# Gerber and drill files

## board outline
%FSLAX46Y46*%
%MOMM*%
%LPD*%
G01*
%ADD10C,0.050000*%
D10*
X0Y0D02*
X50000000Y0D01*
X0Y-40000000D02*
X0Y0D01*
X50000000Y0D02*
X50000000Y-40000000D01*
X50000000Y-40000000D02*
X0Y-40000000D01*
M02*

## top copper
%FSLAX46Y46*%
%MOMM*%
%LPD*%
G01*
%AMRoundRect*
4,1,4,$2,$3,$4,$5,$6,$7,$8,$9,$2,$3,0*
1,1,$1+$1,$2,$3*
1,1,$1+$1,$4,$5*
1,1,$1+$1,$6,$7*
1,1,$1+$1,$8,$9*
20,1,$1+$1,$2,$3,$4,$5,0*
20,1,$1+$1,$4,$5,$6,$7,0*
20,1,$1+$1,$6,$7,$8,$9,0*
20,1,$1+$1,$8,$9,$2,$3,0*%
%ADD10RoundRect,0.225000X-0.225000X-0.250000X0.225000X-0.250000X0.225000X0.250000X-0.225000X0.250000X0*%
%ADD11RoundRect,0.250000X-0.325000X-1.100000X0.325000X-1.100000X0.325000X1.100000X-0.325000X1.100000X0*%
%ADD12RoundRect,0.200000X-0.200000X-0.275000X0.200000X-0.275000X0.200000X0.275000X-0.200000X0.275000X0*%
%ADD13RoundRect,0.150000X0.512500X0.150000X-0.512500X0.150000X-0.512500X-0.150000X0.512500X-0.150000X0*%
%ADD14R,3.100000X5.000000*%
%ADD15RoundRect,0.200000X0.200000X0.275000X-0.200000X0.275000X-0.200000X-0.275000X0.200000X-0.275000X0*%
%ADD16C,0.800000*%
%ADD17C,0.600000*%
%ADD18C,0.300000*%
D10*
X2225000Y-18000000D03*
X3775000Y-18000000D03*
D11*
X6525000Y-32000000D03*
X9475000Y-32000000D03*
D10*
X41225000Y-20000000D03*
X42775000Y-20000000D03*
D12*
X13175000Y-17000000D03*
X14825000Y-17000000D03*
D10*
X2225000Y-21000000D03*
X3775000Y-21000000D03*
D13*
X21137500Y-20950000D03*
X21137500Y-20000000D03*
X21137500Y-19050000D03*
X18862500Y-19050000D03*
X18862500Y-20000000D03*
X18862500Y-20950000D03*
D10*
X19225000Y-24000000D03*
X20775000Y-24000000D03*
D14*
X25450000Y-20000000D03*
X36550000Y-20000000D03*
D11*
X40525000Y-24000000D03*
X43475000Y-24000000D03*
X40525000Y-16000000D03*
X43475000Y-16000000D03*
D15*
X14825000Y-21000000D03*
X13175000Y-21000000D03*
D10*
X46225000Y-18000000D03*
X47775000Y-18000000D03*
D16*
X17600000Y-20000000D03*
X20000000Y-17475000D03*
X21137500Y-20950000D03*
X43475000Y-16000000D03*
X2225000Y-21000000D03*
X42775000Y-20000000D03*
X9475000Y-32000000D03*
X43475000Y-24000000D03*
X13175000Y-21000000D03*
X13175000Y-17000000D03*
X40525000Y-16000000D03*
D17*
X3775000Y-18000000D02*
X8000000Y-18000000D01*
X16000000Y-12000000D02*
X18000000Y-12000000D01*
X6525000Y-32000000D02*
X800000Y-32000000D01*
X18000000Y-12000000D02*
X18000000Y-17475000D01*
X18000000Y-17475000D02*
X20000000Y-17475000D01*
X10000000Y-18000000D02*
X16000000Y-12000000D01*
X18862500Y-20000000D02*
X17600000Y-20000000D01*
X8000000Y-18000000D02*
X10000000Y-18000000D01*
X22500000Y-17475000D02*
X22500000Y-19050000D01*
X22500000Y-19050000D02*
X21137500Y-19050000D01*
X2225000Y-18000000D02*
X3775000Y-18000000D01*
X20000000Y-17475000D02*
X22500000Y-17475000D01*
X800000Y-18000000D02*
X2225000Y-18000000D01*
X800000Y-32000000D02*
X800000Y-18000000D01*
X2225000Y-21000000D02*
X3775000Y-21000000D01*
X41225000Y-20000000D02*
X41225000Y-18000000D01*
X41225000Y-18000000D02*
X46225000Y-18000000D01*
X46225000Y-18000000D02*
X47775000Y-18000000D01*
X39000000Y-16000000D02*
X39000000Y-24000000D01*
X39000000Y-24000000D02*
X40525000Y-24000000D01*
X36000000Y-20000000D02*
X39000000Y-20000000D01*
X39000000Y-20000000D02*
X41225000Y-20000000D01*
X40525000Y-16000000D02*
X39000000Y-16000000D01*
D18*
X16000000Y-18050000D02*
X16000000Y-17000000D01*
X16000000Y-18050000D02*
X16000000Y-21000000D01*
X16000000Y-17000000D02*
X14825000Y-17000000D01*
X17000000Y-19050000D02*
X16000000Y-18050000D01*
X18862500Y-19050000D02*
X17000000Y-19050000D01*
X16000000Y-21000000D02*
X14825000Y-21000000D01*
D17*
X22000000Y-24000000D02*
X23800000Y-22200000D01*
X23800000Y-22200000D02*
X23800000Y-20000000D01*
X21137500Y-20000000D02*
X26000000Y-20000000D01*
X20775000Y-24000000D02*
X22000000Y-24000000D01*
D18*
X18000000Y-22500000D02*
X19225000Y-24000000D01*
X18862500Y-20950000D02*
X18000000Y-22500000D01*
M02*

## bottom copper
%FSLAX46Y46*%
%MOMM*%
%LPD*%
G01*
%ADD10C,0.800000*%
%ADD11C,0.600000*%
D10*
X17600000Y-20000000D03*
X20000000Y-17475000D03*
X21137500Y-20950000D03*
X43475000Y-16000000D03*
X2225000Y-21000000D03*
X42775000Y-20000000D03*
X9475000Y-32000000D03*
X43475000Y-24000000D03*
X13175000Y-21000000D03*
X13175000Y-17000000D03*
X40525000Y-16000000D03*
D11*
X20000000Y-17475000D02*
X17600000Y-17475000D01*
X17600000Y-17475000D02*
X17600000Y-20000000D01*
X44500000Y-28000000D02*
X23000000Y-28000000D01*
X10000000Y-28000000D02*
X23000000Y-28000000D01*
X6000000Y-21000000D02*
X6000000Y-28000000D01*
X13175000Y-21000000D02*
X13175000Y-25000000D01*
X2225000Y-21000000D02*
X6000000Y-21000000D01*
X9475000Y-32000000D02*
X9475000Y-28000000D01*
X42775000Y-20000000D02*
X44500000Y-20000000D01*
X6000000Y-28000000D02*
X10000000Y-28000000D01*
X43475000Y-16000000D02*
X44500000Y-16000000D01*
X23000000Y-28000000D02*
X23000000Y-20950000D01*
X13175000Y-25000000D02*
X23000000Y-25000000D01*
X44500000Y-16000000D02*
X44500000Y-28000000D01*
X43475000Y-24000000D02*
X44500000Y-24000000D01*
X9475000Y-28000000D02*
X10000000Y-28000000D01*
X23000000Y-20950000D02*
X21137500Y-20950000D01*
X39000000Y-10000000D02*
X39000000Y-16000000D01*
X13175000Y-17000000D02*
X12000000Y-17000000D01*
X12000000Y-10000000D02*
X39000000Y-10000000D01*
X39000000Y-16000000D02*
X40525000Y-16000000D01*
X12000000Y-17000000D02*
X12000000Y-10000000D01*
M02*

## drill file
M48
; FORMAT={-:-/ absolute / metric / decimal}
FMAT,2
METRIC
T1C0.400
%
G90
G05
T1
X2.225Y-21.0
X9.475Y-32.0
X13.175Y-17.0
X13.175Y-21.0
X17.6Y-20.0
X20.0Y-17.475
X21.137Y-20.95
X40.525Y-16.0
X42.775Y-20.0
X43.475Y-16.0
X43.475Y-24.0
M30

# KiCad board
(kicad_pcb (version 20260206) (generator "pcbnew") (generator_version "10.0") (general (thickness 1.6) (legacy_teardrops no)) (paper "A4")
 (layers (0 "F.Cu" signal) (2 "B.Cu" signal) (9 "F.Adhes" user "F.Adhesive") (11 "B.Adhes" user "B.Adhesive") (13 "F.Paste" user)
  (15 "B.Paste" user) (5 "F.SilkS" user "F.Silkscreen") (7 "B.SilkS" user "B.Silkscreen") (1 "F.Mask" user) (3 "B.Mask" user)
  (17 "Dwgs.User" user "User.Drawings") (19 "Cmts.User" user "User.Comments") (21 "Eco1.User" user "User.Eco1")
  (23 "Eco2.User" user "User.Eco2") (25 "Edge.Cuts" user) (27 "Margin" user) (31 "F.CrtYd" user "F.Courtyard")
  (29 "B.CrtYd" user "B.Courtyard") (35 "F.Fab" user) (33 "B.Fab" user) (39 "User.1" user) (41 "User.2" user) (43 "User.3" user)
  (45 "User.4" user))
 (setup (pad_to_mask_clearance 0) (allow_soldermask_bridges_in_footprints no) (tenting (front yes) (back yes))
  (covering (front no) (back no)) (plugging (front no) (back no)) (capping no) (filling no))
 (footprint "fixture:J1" (layer "F.Cu") (at 3 18)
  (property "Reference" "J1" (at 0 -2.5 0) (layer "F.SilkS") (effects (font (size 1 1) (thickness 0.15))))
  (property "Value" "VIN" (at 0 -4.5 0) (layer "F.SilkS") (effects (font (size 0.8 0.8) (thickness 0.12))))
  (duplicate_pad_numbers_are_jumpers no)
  (pad "1" smd roundrect (at -0.775 0) (size 0.9 0.95) (layers "F.Cu" "F.Mask" "F.Paste") (roundrect_rratio 0.25) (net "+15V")
   (thermal_bridge_angle 45))
  (pad "2" smd roundrect (at 0.775 0) (size 0.9 0.95) (layers "F.Cu" "F.Mask" "F.Paste") (roundrect_rratio 0.25) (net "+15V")
   (thermal_bridge_angle 45)))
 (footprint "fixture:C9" (layer "F.Cu") (at 8 32)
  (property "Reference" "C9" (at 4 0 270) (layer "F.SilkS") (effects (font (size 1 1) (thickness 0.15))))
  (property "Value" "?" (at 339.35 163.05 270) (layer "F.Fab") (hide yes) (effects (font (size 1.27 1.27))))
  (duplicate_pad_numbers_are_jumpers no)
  (pad "1" smd roundrect (at -1.475 0) (size 1.15 2.7) (layers "F.Cu" "F.Mask" "F.Paste") (roundrect_rratio 0.217391) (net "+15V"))
  (pad "2" smd roundrect (at 1.475 0) (size 1.15 2.7) (layers "F.Cu" "F.Mask" "F.Paste") (roundrect_rratio 0.217391) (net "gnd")))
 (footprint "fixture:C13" (layer "F.Cu") (at 42 20)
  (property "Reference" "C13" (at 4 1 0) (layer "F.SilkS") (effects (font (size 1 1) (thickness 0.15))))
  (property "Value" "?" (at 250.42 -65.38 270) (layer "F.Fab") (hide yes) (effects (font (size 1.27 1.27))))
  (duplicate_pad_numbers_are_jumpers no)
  (pad "1" smd roundrect (at -0.775 0) (size 0.9 0.95) (layers "F.Cu" "F.Mask" "F.Paste") (roundrect_rratio 0.25) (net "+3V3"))
  (pad "2" smd roundrect (at 0.775 0) (size 0.9 0.95) (layers "F.Cu" "F.Mask" "F.Paste") (roundrect_rratio 0.25) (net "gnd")))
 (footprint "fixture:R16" (layer "F.Cu") (at 14 17)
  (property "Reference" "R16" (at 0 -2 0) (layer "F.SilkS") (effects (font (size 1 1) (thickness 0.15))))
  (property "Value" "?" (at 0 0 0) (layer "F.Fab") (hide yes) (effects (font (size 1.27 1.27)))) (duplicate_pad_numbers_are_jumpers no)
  (pad "1" smd roundrect (at -0.825 0) (size 0.8 0.95) (layers "F.Cu" "F.Mask" "F.Paste") (roundrect_rratio 0.25) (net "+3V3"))
  (pad "2" smd roundrect (at 0.825 0) (size 0.8 0.95) (layers "F.Cu" "F.Mask" "F.Paste") (roundrect_rratio 0.25) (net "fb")))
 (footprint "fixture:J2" (layer "F.Cu") (at 3 21)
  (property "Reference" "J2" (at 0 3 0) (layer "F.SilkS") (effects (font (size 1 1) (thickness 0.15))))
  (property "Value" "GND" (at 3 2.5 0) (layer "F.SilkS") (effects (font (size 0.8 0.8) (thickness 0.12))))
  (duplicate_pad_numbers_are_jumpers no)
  (pad "1" smd roundrect (at -0.775 0) (size 0.9 0.95) (layers "F.Cu" "F.Mask" "F.Paste") (roundrect_rratio 0.25) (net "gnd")
   (thermal_bridge_angle 45))
  (pad "2" smd roundrect (at 0.775 0) (size 0.9 0.95) (layers "F.Cu" "F.Mask" "F.Paste") (roundrect_rratio 0.25) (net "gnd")
   (thermal_bridge_angle 45)))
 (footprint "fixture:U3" (layer "F.Cu") (at 20 20 180)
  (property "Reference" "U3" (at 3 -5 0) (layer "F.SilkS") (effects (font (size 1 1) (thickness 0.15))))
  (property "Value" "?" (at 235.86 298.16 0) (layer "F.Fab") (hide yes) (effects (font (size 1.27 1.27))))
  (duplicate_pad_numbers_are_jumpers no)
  (pad "1" smd roundrect (at -1.1375 -0.95 180) (size 1.325 0.6) (layers "F.Cu" "F.Mask" "F.Paste") (roundrect_rratio 0.25) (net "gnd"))
  (pad "2" smd roundrect (at -1.1375 0 180) (size 1.325 0.6) (layers "F.Cu" "F.Mask" "F.Paste") (roundrect_rratio 0.25) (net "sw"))
  (pad "3" smd roundrect (at -1.1375 0.95 180) (size 1.325 0.6) (layers "F.Cu" "F.Mask" "F.Paste") (roundrect_rratio 0.25) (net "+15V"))
  (pad "4" smd roundrect (at 1.1375 0.95 180) (size 1.325 0.6) (layers "F.Cu" "F.Mask" "F.Paste") (roundrect_rratio 0.25) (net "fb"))
  (pad "5" smd roundrect (at 1.1375 0 180) (size 1.325 0.6) (layers "F.Cu" "F.Mask" "F.Paste") (roundrect_rratio 0.25) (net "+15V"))
  (pad "6" smd roundrect (at 1.1375 -0.95 180) (size 1.325 0.6) (layers "F.Cu" "F.Mask" "F.Paste") (roundrect_rratio 0.25) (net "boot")))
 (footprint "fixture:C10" (layer "F.Cu") (at 20 24)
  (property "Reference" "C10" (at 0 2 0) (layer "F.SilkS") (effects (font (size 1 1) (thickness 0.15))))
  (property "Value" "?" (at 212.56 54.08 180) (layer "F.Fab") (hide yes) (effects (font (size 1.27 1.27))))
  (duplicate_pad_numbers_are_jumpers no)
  (pad "1" smd roundrect (at -0.775 0) (size 0.9 0.95) (layers "F.Cu" "F.Mask" "F.Paste") (roundrect_rratio 0.25) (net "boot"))
  (pad "2" smd roundrect (at 0.775 0) (size 0.9 0.95) (layers "F.Cu" "F.Mask" "F.Paste") (roundrect_rratio 0.25) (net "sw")))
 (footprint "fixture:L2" (layer "F.Cu") (at 31 20)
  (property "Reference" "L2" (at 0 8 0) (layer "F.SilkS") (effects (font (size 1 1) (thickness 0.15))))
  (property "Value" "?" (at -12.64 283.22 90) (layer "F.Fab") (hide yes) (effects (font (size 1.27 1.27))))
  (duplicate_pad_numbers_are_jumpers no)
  (pad "1" smd rect (at -5.55 0) (size 3.1 5) (layers "F.Cu" "F.Mask" "F.Paste") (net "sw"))
  (pad "2" smd rect (at 5.55 0) (size 3.1 5) (layers "F.Cu" "F.Mask" "F.Paste") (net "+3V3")))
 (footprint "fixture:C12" (layer "F.Cu") (at 42 24)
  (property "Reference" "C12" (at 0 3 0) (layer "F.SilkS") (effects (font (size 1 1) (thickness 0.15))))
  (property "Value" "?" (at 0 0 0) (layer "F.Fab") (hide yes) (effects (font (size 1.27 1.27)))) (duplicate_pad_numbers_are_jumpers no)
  (pad "1" smd roundrect (at -1.475 0) (size 1.15 2.7) (layers "F.Cu" "F.Mask" "F.Paste") (roundrect_rratio 0.217391) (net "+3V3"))
  (pad "2" smd roundrect (at 1.475 0) (size 1.15 2.7) (layers "F.Cu" "F.Mask" "F.Paste") (roundrect_rratio 0.217391) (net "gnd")))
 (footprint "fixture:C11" (layer "F.Cu") (at 42 16)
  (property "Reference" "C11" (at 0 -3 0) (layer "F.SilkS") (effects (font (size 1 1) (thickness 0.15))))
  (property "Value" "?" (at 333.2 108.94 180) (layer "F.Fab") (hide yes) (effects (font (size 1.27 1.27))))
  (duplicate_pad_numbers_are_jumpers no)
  (pad "1" smd roundrect (at -1.475 0) (size 1.15 2.7) (layers "F.Cu" "F.Mask" "F.Paste") (roundrect_rratio 0.217391) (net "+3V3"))
  (pad "2" smd roundrect (at 1.475 0) (size 1.15 2.7) (layers "F.Cu" "F.Mask" "F.Paste") (roundrect_rratio 0.217391) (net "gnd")))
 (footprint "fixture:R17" (layer "F.Cu") (at 14 21 180)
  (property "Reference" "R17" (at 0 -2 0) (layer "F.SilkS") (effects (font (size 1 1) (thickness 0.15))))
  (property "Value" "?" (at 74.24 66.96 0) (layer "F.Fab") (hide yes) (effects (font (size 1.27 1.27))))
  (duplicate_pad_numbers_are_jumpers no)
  (pad "1" smd roundrect (at -0.825 0 180) (size 0.8 0.95) (layers "F.Cu" "F.Mask" "F.Paste") (roundrect_rratio 0.25) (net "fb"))
  (pad "2" smd roundrect (at 0.825 0 180) (size 0.8 0.95) (layers "F.Cu" "F.Mask" "F.Paste") (roundrect_rratio 0.25) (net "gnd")))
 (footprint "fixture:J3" (layer "F.Cu") (at 47 18)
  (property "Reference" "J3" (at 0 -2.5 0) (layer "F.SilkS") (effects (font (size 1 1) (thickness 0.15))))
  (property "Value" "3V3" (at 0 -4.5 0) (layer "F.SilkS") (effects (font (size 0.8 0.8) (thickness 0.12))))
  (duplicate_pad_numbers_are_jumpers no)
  (pad "1" smd roundrect (at -0.775 0) (size 0.9 0.95) (layers "F.Cu" "F.Mask" "F.Paste") (roundrect_rratio 0.25) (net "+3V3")
   (thermal_bridge_angle 45))
  (pad "2" smd roundrect (at 0.775 0) (size 0.9 0.95) (layers "F.Cu" "F.Mask" "F.Paste") (roundrect_rratio 0.25) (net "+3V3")
   (thermal_bridge_angle 45)))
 (gr_line (start 0 0) (end 50 0) (stroke (width 0.05) (type default)) (layer "Edge.Cuts"))
 (gr_line (start 0 40) (end 0 0) (stroke (width 0.05) (type default)) (layer "Edge.Cuts"))
 (gr_line (start 50 0) (end 50 40) (stroke (width 0.05) (type default)) (layer "Edge.Cuts"))
 (gr_line (start 50 40) (end 0 40) (stroke (width 0.05) (type default)) (layer "Edge.Cuts"))
 (segment (start 3.775 18) (end 8 18) (width 0.6) (layer "F.Cu") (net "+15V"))
 (segment (start 16 12) (end 18 12) (width 0.6) (layer "F.Cu") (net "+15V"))
 (segment (start 6.525 32) (end 0.8 32) (width 0.6) (layer "F.Cu") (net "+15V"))
 (segment (start 18 12) (end 18 17.475) (width 0.6) (layer "F.Cu") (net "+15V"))
 (segment (start 18 17.475) (end 20 17.475) (width 0.6) (layer "F.Cu") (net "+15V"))
 (segment (start 10 18) (end 16 12) (width 0.6) (layer "F.Cu") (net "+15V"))
 (segment (start 18.8625 20) (end 17.6 20) (width 0.6) (layer "F.Cu") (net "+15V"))
 (segment (start 8 18) (end 10 18) (width 0.6) (layer "F.Cu") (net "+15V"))
 (segment (start 22.5 17.475) (end 22.5 19.05) (width 0.6) (layer "F.Cu") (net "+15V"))
 (segment (start 22.5 19.05) (end 21.1375 19.05) (width 0.6) (layer "F.Cu") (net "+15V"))
 (segment (start 2.225 18) (end 3.775 18) (width 0.6) (layer "F.Cu") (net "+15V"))
 (segment (start 20 17.475) (end 22.5 17.475) (width 0.6) (layer "F.Cu") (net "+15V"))
 (segment (start 0.8 18) (end 2.225 18) (width 0.6) (layer "F.Cu") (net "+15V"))
 (segment (start 0.8 32) (end 0.8 18) (width 0.6) (layer "F.Cu") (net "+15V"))
 (via (at 17.6 20) (size 0.8) (drill 0.4) (layers "F.Cu" "B.Cu") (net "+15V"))
 (via (at 20 17.475) (size 0.8) (drill 0.4) (layers "F.Cu" "B.Cu") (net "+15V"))
 (segment (start 20 17.475) (end 17.6 17.475) (width 0.6) (layer "B.Cu") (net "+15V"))
 (segment (start 17.6 17.475) (end 17.6 20) (width 0.6) (layer "B.Cu") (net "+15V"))
 (segment (start 2.225 21) (end 3.775 21) (width 0.6) (layer "F.Cu") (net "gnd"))
 (via (at 21.1375 20.95) (size 0.8) (drill 0.4) (layers "F.Cu" "B.Cu") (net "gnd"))
 (via (at 43.475 16) (size 0.8) (drill 0.4) (layers "F.Cu" "B.Cu") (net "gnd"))
 (via (at 2.225 21) (size 0.8) (drill 0.4) (layers "F.Cu" "B.Cu") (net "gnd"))
 (via (at 42.775 20) (size 0.8) (drill 0.4) (layers "F.Cu" "B.Cu") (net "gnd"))
 (via (at 9.475 32) (size 0.8) (drill 0.4) (layers "F.Cu" "B.Cu") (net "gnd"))
 (via (at 43.475 24) (size 0.8) (drill 0.4) (layers "F.Cu" "B.Cu") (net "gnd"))
 (via (at 13.175 21) (size 0.8) (drill 0.4) (layers "F.Cu" "B.Cu") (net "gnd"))
 (segment (start 44.5 28) (end 23 28) (width 0.6) (layer "B.Cu") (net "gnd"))
 (segment (start 10 28) (end 23 28) (width 0.6) (layer "B.Cu") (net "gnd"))
 (segment (start 6 21) (end 6 28) (width 0.6) (layer "B.Cu") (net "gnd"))
 (segment (start 13.175 21) (end 13.175 25) (width 0.6) (layer "B.Cu") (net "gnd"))
 (segment (start 2.225 21) (end 6 21) (width 0.6) (layer "B.Cu") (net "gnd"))
 (segment (start 9.475 32) (end 9.475 28) (width 0.6) (layer "B.Cu") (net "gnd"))
 (segment (start 42.775 20) (end 44.5 20) (width 0.6) (layer "B.Cu") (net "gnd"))
 (segment (start 6 28) (end 10 28) (width 0.6) (layer "B.Cu") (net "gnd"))
 (segment (start 43.475 16) (end 44.5 16) (width 0.6) (layer "B.Cu") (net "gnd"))
 (segment (start 23 28) (end 23 20.95) (width 0.6) (layer "B.Cu") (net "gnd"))
 (segment (start 13.175 25) (end 23 25) (width 0.6) (layer "B.Cu") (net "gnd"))
 (segment (start 44.5 16) (end 44.5 28) (width 0.6) (layer "B.Cu") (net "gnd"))
 (segment (start 43.475 24) (end 44.5 24) (width 0.6) (layer "B.Cu") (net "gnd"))
 (segment (start 9.475 28) (end 10 28) (width 0.6) (layer "B.Cu") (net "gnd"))
 (segment (start 23 20.95) (end 21.1375 20.95) (width 0.6) (layer "B.Cu") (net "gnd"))
 (segment (start 41.225 20) (end 41.225 18) (width 0.6) (layer "F.Cu") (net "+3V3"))
 (segment (start 41.225 18) (end 46.225 18) (width 0.6) (layer "F.Cu") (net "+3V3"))
 (segment (start 46.225 18) (end 47.775 18) (width 0.6) (layer "F.Cu") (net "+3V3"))
 (segment (start 39 16) (end 39 24) (width 0.6) (layer "F.Cu") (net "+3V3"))
 (segment (start 39 24) (end 40.525 24) (width 0.6) (layer "F.Cu") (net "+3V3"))
 (segment (start 36 20) (end 39 20) (width 0.6) (layer "F.Cu") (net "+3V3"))
 (segment (start 39 20) (end 41.225 20) (width 0.6) (layer "F.Cu") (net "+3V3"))
 (segment (start 40.525 16) (end 39 16) (width 0.6) (layer "F.Cu") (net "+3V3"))
 (via (at 13.175 17) (size 0.8) (drill 0.4) (layers "F.Cu" "B.Cu") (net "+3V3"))
 (via (at 40.525 16) (size 0.8) (drill 0.4) (layers "F.Cu" "B.Cu") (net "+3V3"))
 (segment (start 39 10) (end 39 16) (width 0.6) (layer "B.Cu") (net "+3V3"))
 (segment (start 13.175 17) (end 12 17) (width 0.6) (layer "B.Cu") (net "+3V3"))
 (segment (start 12 10) (end 39 10) (width 0.6) (layer "B.Cu") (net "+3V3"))
 (segment (start 39 16) (end 40.525 16) (width 0.6) (layer "B.Cu") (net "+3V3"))
 (segment (start 12 17) (end 12 10) (width 0.6) (layer "B.Cu") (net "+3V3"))
 (segment (start 16 18.05) (end 16 17) (width 0.3) (layer "F.Cu") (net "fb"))
 (segment (start 16 18.05) (end 16 21) (width 0.3) (layer "F.Cu") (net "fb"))
 (segment (start 16 17) (end 14.825 17) (width 0.3) (layer "F.Cu") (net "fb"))
 (segment (start 17 19.05) (end 16 18.05) (width 0.3) (layer "F.Cu") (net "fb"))
 (segment (start 18.8625 19.05) (end 17 19.05) (width 0.3) (layer "F.Cu") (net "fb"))
 (segment (start 16 21) (end 14.825 21) (width 0.3) (layer "F.Cu") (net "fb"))
 (segment (start 22 24) (end 23.8 22.2) (width 0.6) (layer "F.Cu") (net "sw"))
 (segment (start 23.8 22.2) (end 23.8 20) (width 0.6) (layer "F.Cu") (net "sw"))
 (segment (start 21.1375 20) (end 26 20) (width 0.6) (layer "F.Cu") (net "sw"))
 (segment (start 20.775 24) (end 22 24) (width 0.6) (layer "F.Cu") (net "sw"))
 (segment (start 18 22.5) (end 19.225 24) (width 0.3) (layer "F.Cu") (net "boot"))
 (segment (start 18.8625 20.95) (end 18 22.5) (width 0.3) (layer "F.Cu") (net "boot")))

